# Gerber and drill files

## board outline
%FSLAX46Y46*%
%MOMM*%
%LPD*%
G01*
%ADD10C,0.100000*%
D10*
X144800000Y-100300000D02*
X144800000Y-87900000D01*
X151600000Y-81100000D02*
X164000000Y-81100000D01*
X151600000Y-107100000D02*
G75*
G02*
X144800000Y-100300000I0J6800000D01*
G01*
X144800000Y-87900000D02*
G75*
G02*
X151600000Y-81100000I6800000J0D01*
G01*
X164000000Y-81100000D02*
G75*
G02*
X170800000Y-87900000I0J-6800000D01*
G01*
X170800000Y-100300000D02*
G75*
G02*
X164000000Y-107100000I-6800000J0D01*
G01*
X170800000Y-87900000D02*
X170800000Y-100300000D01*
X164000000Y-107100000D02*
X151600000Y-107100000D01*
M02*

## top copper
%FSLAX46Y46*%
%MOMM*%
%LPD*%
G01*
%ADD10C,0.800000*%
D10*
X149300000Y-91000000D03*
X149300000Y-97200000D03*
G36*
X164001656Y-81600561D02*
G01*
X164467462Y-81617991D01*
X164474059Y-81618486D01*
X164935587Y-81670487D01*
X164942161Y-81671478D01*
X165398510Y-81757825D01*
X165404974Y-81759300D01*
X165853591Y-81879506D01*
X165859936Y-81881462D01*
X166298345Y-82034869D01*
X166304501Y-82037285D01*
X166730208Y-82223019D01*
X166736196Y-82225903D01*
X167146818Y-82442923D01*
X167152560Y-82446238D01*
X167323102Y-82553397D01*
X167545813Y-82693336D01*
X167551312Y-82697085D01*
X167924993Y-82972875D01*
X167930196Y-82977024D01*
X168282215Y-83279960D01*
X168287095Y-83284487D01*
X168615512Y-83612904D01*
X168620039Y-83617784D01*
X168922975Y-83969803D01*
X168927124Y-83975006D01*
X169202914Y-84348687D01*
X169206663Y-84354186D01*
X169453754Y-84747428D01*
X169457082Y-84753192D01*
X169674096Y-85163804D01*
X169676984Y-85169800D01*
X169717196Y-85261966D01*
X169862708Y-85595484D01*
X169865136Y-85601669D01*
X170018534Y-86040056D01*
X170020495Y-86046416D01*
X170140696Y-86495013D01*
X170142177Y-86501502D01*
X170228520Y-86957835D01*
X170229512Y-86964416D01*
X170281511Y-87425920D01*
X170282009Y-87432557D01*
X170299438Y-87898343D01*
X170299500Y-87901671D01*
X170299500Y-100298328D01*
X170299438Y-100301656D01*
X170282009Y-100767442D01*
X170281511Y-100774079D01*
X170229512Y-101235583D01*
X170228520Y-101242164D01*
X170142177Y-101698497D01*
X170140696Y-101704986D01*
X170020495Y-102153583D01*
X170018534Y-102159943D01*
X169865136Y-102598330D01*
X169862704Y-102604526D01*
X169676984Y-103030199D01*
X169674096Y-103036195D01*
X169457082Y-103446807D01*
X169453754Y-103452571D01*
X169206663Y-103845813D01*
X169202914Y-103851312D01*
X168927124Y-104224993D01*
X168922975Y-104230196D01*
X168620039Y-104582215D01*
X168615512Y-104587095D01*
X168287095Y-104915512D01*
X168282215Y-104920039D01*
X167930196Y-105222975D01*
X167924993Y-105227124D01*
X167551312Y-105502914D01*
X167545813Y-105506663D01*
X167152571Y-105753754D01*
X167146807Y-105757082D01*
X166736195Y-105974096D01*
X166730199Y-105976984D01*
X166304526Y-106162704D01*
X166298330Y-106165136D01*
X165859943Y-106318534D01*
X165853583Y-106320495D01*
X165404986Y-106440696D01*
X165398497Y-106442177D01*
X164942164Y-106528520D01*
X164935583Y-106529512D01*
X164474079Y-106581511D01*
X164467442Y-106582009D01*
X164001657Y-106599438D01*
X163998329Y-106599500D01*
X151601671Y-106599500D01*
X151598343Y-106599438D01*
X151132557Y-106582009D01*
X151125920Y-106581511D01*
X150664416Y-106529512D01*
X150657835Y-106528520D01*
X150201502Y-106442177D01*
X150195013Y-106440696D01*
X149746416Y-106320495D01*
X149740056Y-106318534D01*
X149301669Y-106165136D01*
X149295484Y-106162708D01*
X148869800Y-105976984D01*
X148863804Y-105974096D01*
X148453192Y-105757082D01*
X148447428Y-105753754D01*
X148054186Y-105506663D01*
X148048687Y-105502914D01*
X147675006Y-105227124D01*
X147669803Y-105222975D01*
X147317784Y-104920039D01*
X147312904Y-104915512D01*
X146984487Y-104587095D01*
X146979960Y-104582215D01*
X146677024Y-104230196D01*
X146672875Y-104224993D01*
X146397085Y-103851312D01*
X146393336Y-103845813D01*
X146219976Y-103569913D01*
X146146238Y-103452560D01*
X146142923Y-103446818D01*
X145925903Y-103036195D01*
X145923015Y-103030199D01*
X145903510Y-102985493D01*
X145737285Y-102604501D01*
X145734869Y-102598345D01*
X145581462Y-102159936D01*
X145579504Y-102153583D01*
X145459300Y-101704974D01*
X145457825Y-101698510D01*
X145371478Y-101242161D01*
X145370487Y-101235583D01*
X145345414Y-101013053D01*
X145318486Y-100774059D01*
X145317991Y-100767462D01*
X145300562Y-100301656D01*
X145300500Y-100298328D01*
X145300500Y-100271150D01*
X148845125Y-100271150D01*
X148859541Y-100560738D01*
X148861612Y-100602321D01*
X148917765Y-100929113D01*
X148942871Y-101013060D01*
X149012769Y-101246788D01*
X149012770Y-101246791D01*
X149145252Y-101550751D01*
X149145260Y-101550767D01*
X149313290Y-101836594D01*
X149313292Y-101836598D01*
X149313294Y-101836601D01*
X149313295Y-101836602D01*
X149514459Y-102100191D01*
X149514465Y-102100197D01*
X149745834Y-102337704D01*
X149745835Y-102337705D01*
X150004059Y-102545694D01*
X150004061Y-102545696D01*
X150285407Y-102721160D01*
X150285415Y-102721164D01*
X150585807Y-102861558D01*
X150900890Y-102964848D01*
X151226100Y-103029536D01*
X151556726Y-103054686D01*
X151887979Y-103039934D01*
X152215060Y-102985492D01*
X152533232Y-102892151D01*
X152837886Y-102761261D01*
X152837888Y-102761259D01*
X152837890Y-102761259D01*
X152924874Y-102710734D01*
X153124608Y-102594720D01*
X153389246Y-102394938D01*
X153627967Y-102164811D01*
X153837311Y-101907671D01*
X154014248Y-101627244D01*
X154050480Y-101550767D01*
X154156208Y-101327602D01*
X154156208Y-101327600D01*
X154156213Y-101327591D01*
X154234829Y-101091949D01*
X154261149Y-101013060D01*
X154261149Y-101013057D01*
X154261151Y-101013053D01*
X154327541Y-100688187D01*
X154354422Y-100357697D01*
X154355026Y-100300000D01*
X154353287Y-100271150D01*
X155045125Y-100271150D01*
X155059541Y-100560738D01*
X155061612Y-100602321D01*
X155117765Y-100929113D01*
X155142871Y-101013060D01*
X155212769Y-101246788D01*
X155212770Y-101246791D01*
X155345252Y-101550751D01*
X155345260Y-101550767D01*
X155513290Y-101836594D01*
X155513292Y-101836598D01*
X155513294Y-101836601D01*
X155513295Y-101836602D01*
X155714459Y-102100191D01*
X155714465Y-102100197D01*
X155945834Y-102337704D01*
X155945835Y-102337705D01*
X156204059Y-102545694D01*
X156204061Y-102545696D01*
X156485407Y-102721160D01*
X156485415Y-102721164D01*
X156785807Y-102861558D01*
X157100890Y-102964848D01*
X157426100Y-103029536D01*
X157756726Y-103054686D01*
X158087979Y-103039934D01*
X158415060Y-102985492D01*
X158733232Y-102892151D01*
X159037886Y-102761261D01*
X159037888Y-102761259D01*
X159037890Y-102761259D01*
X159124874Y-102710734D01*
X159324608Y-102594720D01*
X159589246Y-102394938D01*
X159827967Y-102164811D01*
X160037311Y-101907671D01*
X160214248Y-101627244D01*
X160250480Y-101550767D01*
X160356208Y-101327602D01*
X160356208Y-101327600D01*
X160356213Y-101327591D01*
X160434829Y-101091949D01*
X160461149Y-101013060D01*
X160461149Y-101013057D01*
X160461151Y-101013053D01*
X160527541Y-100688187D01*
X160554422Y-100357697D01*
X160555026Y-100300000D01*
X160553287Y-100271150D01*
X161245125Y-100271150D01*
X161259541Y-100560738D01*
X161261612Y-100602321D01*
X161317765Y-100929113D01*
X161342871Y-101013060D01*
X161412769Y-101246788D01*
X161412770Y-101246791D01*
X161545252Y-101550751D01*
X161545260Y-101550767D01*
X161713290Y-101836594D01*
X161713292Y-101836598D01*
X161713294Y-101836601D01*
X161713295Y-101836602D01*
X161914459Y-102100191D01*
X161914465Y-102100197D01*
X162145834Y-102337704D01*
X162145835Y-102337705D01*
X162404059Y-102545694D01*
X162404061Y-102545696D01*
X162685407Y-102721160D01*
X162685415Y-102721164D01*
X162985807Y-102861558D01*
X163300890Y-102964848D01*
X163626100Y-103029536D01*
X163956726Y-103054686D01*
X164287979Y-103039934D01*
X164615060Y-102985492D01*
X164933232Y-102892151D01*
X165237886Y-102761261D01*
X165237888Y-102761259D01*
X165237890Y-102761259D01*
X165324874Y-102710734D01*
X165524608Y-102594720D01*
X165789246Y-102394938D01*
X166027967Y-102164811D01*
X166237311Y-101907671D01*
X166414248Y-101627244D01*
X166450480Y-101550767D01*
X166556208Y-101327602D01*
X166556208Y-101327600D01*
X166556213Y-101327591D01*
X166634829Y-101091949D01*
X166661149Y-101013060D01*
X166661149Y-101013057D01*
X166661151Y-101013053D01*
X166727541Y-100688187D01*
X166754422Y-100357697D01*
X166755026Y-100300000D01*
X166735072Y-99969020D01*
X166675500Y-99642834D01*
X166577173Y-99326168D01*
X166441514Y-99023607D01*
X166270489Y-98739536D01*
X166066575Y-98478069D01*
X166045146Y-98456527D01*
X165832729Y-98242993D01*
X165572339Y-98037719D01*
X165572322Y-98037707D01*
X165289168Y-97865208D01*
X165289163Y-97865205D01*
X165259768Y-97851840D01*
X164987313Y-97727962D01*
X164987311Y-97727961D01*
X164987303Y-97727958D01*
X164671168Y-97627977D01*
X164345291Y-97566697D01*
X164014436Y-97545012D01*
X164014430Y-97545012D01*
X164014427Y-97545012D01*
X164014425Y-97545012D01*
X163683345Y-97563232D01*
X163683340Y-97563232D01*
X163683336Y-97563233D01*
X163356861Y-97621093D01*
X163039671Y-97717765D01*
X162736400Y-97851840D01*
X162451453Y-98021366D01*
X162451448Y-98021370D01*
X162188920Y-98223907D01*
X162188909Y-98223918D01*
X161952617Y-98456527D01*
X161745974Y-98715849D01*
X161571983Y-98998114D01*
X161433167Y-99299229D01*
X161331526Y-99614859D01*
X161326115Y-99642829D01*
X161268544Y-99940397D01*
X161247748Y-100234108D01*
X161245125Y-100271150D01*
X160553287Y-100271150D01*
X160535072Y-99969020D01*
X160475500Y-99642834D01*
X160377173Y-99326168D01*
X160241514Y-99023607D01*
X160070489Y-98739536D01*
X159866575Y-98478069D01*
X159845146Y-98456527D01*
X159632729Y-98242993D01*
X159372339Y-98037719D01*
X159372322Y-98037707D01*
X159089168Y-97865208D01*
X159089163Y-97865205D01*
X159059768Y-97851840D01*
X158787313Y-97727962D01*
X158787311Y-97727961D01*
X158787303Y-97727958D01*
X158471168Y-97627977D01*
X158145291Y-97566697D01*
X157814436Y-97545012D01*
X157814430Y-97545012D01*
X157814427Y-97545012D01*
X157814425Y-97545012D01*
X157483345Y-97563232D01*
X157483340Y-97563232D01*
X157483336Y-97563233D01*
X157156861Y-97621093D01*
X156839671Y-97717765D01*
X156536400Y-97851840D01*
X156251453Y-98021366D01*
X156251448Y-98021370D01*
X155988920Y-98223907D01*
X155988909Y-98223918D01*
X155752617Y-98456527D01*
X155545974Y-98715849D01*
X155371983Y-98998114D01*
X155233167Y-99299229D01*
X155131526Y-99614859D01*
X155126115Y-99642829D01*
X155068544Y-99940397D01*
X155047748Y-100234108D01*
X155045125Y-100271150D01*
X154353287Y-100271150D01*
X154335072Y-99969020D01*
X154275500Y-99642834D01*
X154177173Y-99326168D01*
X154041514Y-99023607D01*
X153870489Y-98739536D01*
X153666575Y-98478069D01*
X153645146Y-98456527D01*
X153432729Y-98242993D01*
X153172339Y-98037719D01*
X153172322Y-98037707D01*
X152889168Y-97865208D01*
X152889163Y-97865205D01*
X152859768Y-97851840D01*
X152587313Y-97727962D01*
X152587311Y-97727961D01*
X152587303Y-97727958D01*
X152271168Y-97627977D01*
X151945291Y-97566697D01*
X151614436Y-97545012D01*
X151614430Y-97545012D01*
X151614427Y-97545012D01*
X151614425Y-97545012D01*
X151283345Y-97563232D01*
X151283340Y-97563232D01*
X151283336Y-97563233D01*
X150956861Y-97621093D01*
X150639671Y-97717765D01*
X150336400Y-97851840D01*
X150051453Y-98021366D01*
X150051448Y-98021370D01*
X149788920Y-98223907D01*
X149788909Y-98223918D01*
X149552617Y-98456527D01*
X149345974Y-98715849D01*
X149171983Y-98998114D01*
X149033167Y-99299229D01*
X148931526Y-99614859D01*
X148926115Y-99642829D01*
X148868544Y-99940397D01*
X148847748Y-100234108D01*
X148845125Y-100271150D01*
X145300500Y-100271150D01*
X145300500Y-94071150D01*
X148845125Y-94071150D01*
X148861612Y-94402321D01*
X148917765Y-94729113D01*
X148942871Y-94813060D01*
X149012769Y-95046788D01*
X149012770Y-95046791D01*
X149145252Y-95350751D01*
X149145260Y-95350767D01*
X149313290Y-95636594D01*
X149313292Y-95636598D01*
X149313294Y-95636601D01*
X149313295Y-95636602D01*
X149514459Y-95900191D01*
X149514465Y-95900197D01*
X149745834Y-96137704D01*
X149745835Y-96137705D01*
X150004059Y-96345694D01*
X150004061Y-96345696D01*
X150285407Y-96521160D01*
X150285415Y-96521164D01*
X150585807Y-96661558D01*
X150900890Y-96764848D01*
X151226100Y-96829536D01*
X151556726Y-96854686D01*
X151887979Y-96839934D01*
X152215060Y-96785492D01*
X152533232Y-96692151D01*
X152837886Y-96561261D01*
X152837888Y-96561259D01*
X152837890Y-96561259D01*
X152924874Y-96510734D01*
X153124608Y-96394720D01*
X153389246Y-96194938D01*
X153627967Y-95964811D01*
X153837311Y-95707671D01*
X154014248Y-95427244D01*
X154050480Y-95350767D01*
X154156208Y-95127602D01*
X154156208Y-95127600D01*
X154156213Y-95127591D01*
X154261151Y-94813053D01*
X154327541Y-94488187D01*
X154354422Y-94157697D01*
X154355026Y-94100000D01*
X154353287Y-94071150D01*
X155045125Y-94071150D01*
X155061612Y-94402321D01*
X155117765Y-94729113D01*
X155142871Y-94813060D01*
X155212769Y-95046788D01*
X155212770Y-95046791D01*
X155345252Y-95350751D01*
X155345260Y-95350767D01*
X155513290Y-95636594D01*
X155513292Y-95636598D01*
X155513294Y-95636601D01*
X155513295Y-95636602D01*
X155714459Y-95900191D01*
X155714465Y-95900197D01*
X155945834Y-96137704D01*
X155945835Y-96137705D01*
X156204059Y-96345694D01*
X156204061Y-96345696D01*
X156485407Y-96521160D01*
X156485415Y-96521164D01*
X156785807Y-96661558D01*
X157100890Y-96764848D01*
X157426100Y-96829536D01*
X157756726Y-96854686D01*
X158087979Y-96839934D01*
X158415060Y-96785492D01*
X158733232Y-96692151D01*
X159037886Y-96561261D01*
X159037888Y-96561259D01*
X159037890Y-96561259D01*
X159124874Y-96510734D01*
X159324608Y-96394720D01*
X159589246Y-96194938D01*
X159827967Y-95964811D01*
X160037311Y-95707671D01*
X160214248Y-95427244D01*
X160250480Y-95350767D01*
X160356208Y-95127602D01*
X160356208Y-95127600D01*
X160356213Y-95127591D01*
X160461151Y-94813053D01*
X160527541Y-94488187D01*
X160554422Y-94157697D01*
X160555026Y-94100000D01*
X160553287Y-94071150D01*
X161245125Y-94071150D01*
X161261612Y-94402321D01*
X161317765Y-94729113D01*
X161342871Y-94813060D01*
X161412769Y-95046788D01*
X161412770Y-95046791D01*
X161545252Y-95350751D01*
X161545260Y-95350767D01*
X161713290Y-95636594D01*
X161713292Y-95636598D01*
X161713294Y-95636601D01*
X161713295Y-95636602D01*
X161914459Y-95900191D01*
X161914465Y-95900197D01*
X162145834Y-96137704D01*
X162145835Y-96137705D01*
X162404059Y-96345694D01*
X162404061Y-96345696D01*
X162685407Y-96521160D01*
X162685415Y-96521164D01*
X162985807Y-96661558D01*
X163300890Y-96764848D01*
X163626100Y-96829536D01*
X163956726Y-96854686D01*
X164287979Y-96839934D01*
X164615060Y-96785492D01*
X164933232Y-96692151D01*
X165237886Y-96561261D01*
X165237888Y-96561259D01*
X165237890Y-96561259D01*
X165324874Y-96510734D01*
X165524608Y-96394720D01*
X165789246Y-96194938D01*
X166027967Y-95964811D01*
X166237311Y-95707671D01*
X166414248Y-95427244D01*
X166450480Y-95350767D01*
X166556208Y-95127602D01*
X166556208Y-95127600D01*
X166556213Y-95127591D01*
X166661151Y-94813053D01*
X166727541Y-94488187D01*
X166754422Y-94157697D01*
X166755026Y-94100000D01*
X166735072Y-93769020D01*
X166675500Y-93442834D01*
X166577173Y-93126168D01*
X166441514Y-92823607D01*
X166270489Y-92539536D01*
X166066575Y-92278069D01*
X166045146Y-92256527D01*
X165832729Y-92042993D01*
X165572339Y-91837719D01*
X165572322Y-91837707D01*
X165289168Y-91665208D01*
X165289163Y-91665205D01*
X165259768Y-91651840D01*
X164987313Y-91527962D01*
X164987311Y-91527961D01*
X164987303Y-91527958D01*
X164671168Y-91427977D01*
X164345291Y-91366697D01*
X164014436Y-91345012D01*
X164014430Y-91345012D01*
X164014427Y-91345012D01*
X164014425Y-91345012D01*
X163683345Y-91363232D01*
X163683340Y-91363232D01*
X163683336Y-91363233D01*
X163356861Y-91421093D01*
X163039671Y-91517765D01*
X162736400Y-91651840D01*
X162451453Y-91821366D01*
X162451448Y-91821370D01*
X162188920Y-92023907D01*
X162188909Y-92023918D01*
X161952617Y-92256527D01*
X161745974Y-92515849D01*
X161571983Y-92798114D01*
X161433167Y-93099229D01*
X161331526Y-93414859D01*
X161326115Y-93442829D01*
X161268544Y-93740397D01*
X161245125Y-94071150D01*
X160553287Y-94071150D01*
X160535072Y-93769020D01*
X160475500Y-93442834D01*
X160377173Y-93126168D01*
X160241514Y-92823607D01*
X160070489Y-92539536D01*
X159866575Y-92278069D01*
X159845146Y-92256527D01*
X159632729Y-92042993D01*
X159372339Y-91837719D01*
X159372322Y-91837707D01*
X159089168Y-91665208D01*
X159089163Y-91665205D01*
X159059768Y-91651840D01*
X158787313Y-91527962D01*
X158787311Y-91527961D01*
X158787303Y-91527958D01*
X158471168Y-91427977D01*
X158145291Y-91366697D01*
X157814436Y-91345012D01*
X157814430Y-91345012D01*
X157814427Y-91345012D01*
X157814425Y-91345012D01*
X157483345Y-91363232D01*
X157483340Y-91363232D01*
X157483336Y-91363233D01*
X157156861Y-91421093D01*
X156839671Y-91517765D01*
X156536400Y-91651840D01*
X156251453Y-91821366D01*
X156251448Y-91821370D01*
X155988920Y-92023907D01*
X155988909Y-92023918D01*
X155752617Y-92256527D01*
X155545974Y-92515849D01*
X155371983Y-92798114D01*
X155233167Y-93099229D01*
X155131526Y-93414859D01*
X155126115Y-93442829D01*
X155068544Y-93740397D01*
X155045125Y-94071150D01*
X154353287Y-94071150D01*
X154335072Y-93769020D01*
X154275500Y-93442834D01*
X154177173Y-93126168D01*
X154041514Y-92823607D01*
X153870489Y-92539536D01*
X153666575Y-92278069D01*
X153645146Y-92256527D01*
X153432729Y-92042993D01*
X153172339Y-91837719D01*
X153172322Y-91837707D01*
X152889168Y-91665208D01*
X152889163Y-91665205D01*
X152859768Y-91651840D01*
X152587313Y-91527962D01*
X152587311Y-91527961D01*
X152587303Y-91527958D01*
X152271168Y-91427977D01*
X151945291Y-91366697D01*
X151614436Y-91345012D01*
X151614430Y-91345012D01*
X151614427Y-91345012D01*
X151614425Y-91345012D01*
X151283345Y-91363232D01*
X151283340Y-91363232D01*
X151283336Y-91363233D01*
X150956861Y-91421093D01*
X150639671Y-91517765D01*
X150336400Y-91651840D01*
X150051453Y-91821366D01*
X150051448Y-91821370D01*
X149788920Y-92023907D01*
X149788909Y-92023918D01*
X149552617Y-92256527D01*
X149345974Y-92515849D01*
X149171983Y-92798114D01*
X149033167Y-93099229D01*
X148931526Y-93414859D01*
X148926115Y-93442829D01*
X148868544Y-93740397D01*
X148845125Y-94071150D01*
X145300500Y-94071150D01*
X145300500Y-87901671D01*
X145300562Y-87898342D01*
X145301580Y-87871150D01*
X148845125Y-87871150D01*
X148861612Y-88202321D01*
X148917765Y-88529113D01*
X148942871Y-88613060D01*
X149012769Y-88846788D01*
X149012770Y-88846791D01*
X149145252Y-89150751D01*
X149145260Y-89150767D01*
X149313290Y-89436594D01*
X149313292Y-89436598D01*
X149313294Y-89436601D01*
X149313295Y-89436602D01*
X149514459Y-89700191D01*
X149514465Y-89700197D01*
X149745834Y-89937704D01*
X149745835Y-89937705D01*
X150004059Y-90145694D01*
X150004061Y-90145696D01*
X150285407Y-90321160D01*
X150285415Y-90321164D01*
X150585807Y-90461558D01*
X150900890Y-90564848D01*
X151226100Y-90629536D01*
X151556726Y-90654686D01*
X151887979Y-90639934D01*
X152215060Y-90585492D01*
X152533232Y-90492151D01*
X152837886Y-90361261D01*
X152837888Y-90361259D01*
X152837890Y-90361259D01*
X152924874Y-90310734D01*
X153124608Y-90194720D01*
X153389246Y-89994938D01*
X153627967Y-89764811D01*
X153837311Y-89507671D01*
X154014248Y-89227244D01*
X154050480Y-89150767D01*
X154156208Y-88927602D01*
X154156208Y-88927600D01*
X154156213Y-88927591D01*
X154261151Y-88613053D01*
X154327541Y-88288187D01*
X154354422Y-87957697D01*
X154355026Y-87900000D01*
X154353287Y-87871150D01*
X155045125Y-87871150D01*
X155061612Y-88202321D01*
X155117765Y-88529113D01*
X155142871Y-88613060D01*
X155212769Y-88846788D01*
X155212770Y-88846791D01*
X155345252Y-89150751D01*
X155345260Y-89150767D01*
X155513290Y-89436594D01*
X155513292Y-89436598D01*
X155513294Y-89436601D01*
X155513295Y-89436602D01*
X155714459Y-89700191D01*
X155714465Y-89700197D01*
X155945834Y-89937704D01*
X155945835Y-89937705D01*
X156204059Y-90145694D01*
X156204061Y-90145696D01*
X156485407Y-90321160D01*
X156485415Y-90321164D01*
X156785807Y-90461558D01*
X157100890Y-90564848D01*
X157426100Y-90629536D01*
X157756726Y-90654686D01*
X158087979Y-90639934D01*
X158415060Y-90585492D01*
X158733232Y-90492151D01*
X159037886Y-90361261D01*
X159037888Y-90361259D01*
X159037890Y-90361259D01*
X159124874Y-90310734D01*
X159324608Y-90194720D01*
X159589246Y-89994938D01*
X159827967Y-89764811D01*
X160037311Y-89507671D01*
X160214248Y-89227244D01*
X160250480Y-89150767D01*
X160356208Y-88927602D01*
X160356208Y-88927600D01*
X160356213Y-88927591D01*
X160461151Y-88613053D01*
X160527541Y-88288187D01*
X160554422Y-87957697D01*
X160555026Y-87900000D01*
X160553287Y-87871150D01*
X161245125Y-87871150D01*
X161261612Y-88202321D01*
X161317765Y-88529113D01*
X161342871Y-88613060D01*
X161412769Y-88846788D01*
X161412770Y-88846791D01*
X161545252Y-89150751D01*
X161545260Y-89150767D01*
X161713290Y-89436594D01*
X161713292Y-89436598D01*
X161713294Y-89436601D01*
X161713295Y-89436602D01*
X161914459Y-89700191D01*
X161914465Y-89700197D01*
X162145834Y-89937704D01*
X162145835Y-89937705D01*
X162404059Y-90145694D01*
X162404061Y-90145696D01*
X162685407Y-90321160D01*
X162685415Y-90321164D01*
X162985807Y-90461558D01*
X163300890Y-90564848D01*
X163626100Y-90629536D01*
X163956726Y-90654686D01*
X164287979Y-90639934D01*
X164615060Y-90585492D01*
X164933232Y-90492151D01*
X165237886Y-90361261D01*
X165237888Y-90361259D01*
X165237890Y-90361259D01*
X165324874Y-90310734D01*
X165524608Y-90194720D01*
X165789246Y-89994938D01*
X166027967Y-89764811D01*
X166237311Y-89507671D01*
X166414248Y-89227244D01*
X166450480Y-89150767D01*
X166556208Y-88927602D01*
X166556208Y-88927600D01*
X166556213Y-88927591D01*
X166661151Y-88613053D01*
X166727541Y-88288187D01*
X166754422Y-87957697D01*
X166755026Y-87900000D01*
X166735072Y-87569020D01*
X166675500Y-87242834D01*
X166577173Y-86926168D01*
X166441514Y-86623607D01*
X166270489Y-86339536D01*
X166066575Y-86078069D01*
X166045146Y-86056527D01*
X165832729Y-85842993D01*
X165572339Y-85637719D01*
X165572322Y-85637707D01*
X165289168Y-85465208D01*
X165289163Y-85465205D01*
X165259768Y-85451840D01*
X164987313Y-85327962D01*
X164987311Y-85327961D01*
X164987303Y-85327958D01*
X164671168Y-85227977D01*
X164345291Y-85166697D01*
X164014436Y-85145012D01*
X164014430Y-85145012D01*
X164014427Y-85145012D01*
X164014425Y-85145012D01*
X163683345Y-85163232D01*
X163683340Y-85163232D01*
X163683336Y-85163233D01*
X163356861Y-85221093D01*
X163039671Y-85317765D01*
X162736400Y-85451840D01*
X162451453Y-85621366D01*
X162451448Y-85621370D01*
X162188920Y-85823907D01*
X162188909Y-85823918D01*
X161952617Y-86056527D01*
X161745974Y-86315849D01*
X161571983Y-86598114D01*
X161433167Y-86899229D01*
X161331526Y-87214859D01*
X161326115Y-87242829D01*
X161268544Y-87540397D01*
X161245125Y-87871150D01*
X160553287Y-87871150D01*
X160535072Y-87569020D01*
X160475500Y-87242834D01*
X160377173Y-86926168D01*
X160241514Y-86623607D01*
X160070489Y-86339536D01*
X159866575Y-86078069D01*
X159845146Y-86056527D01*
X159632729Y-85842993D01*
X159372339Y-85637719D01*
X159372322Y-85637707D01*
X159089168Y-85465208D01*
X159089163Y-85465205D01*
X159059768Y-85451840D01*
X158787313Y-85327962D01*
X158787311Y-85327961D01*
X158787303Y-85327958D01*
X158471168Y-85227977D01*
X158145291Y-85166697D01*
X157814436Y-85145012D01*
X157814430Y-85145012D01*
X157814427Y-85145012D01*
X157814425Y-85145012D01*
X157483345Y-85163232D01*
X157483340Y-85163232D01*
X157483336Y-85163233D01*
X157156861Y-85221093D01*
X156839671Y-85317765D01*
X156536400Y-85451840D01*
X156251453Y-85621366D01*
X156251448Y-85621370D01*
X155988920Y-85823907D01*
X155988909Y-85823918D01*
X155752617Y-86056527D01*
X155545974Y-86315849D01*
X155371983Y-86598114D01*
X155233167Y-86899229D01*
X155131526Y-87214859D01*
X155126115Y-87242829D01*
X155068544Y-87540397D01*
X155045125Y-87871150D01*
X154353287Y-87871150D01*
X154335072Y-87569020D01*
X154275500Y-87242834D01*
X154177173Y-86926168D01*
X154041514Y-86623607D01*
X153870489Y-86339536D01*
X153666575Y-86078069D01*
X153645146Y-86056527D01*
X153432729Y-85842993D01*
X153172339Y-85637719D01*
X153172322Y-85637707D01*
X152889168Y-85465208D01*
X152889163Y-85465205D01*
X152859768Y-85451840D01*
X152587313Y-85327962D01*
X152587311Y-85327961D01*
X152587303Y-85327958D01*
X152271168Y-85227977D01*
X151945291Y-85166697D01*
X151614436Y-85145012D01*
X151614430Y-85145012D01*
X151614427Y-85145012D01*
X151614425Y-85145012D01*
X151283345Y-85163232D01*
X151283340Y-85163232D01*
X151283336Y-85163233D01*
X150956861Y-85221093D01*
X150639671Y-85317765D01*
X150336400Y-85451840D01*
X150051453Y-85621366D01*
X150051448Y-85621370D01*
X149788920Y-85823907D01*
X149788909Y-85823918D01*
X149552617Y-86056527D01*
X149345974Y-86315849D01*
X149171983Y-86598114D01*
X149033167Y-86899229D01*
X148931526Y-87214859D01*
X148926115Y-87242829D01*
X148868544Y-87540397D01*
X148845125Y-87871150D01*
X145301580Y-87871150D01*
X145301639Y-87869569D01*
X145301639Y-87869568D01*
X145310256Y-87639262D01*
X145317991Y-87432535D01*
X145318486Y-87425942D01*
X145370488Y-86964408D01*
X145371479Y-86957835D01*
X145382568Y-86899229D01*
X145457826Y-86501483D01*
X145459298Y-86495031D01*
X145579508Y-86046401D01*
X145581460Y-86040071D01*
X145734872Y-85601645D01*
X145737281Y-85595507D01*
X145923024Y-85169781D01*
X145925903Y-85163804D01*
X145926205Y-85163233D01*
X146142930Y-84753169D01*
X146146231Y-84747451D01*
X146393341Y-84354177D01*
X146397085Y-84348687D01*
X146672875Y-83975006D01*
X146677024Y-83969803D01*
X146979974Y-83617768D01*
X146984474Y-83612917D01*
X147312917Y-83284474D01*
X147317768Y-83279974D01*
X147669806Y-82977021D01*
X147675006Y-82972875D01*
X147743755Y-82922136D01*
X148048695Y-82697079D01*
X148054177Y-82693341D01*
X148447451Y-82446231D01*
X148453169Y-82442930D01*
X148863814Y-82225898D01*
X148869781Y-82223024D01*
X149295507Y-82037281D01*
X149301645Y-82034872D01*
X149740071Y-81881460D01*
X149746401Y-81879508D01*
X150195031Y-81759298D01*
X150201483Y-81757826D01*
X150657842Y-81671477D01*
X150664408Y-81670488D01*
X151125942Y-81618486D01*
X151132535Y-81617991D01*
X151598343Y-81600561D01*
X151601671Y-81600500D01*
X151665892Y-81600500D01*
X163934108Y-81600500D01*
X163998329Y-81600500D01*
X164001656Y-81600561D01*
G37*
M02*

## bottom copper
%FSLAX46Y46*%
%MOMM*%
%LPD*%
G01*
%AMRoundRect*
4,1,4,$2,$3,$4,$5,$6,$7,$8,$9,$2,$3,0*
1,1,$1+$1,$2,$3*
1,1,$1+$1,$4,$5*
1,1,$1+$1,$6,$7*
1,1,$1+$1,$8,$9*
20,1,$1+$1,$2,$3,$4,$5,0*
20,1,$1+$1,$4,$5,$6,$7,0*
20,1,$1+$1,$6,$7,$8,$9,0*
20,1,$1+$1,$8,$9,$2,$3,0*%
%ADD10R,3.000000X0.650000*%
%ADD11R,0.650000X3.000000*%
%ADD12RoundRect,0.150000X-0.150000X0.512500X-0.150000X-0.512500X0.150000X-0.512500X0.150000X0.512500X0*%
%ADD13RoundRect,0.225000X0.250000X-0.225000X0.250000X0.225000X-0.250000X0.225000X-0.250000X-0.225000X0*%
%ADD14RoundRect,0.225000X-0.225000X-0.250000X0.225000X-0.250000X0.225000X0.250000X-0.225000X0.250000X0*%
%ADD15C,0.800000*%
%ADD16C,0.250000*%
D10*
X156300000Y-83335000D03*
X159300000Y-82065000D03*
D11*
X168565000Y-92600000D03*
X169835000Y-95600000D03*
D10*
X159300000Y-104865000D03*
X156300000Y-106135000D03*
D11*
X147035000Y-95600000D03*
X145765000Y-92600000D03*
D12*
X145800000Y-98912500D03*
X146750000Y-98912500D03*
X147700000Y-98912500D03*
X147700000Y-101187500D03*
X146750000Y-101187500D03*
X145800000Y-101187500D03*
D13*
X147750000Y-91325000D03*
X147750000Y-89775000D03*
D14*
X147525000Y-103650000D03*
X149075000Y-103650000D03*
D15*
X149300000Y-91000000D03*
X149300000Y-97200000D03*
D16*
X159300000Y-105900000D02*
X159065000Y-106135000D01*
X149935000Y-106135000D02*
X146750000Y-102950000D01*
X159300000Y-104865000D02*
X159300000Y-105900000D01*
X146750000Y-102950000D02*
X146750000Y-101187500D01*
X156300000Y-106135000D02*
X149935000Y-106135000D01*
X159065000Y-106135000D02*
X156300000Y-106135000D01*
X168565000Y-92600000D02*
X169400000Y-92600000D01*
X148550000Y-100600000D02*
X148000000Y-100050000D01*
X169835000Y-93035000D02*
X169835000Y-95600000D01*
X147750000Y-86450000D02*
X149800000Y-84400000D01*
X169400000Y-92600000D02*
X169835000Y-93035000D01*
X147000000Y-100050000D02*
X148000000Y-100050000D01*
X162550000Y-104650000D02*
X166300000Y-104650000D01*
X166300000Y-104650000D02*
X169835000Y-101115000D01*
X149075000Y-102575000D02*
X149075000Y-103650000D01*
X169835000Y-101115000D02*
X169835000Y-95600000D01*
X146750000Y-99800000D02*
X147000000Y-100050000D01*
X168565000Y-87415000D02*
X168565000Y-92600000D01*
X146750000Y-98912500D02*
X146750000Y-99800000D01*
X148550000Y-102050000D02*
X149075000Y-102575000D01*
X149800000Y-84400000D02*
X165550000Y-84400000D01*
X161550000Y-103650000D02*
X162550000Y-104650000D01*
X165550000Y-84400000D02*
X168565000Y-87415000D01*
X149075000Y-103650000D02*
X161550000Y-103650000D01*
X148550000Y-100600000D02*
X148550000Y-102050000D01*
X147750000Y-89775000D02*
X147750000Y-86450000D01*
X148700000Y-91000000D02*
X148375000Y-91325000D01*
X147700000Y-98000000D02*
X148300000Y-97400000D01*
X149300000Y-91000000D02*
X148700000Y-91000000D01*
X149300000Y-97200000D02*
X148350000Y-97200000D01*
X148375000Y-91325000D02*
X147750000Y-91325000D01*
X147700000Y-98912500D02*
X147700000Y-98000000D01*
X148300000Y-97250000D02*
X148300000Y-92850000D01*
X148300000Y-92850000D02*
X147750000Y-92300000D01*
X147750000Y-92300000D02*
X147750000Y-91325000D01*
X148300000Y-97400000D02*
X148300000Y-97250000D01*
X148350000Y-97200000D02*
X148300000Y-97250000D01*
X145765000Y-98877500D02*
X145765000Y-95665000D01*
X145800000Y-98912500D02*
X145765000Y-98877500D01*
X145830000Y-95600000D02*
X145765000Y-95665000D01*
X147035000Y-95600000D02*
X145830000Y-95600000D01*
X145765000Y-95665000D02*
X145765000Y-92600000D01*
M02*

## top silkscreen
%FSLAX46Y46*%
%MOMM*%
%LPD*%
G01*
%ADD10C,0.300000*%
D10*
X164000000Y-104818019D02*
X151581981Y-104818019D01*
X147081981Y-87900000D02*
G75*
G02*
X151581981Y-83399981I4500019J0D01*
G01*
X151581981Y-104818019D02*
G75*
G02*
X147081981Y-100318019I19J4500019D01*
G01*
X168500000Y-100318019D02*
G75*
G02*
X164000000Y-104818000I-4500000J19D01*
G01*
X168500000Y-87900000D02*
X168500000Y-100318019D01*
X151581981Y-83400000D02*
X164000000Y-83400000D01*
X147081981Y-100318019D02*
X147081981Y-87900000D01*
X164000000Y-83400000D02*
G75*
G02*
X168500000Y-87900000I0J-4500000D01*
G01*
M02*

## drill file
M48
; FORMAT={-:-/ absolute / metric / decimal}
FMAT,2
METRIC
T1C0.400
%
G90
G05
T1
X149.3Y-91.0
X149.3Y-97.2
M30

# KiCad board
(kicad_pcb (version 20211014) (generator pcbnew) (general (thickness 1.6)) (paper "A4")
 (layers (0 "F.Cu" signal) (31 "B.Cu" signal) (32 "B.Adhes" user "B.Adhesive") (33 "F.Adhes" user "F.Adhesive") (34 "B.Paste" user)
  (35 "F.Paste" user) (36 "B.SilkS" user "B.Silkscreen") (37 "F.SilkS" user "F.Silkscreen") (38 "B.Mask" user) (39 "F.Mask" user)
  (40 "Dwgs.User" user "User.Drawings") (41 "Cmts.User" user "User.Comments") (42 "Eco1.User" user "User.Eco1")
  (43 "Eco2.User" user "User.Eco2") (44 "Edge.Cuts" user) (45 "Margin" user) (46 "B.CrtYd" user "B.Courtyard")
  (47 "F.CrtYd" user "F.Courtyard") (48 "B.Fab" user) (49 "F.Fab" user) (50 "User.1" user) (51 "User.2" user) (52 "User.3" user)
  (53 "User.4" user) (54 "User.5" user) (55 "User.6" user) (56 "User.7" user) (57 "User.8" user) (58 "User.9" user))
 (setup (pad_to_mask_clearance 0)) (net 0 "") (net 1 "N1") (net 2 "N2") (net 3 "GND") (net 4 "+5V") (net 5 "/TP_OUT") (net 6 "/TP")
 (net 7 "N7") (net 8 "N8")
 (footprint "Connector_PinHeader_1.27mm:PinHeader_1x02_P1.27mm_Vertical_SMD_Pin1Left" (layer "B.Cu") (at 157.8 82.7)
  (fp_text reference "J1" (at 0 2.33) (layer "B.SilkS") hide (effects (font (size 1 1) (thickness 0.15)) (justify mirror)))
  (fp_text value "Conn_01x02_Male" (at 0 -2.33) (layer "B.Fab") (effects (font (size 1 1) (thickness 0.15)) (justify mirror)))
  (pad "1" smd rect (at -1.5 0.635) (size 3 0.65) (layers "B.Cu" "B.Paste" "B.Mask") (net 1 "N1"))
  (pad "2" smd rect (at 1.5 -0.635) (size 3 0.65) (layers "B.Cu" "B.Paste" "B.Mask") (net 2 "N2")))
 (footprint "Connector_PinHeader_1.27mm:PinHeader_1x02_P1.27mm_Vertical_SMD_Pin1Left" (layer "B.Cu") (at 169.2 94.1 -90)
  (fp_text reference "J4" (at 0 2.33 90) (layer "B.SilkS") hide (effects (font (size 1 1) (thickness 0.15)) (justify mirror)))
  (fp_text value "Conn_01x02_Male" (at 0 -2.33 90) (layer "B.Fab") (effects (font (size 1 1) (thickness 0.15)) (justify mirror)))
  (pad "1" smd rect (at -1.5 0.635 270) (size 3 0.65) (layers "B.Cu" "B.Paste" "B.Mask") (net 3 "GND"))
  (pad "2" smd rect (at 1.5 -0.635 270) (size 3 0.65) (layers "B.Cu" "B.Paste" "B.Mask") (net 3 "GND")))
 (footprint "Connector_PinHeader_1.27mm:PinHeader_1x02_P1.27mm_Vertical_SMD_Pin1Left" (layer "B.Cu") (at 157.8 105.5 180)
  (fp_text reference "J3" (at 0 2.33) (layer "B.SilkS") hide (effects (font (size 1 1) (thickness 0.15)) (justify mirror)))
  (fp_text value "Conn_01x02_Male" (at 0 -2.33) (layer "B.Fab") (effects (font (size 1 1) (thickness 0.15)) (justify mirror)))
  (pad "1" smd rect (at -1.5 0.635 180) (size 3 0.65) (layers "B.Cu" "B.Paste" "B.Mask") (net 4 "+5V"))
  (pad "2" smd rect (at 1.5 -0.635 180) (size 3 0.65) (layers "B.Cu" "B.Paste" "B.Mask") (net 4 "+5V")))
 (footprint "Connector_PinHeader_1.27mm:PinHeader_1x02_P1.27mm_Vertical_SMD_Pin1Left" (layer "B.Cu") (at 146.4 94.1 90)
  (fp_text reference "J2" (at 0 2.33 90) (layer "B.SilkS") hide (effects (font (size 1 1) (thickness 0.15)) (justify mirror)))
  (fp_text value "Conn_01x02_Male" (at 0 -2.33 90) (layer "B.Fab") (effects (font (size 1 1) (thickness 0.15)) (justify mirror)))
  (pad "1" smd rect (at -1.5 0.635 90) (size 3 0.65) (layers "B.Cu" "B.Paste" "B.Mask") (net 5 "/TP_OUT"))
  (pad "2" smd rect (at 1.5 -0.635 90) (size 3 0.65) (layers "B.Cu" "B.Paste" "B.Mask") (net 5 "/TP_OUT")))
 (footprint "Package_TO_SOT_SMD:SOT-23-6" (layer "B.Cu") (at 146.75 100.05 -90)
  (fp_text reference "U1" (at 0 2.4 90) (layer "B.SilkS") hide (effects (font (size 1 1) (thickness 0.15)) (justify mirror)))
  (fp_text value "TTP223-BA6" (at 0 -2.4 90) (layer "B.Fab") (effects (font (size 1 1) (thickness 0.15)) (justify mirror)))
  (pad "1" smd roundrect (at -1.1375 0.95 270) (size 1.325 0.6) (layers "B.Cu" "B.Paste" "B.Mask") (roundrect_rratio 0.25) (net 5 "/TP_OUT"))
  (pad "2" smd roundrect (at -1.1375 0 270) (size 1.325 0.6) (layers "B.Cu" "B.Paste" "B.Mask") (roundrect_rratio 0.25) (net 3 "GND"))
  (pad "3" smd roundrect (at -1.1375 -0.95 270) (size 1.325 0.6) (layers "B.Cu" "B.Paste" "B.Mask") (roundrect_rratio 0.25) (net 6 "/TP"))
  (pad "4" smd roundrect (at 1.1375 -0.95 270) (size 1.325 0.6) (layers "B.Cu" "B.Paste" "B.Mask") (roundrect_rratio 0.25) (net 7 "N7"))
  (pad "5" smd roundrect (at 1.1375 0 270) (size 1.325 0.6) (layers "B.Cu" "B.Paste" "B.Mask") (roundrect_rratio 0.25) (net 4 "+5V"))
  (pad "6" smd roundrect (at 1.1375 0.95 270) (size 1.325 0.6) (layers "B.Cu" "B.Paste" "B.Mask") (roundrect_rratio 0.25) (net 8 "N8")))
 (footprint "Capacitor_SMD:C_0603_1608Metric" (layer "B.Cu") (at 147.75 90.55 90)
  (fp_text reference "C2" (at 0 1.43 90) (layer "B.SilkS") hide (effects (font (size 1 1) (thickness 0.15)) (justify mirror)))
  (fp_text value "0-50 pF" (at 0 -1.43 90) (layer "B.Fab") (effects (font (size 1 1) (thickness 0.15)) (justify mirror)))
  (pad "1" smd roundrect (at -0.775 0 90) (size 0.9 0.95) (layers "B.Cu" "B.Paste" "B.Mask") (roundrect_rratio 0.25) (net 6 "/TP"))
  (pad "2" smd roundrect (at 0.775 0 90) (size 0.9 0.95) (layers "B.Cu" "B.Paste" "B.Mask") (roundrect_rratio 0.25) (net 3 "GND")))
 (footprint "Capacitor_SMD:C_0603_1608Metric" (layer "B.Cu") (at 148.3 103.65)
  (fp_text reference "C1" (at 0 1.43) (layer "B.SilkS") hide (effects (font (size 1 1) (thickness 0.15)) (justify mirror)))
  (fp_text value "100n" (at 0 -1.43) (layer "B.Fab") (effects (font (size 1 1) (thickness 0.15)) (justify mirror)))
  (pad "1" smd roundrect (at -0.775 0) (size 0.9 0.95) (layers "B.Cu" "B.Paste" "B.Mask") (roundrect_rratio 0.25) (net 4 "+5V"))
  (pad "2" smd roundrect (at 0.775 0) (size 0.9 0.95) (layers "B.Cu" "B.Paste" "B.Mask") (roundrect_rratio 0.25) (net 3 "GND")))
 (gr_line (start 164 104.818019) (end 151.581981 104.818019) (layer "F.SilkS") (width 0.3))
 (gr_arc (start 147.081981 87.9) (mid 148.399999 84.718013) (end 151.581981 83.4) (layer "F.SilkS") (width 0.3))
 (gr_arc (start 151.581981 104.818019) (mid 148.400006 103.499994) (end 147.081981 100.318019) (layer "F.SilkS") (width 0.3))
 (gr_arc (start 168.5 100.318019) (mid 167.181981 103.5) (end 164 104.818019) (layer "F.SilkS") (width 0.3))
 (gr_line (start 168.5 87.9) (end 168.5 100.318019) (layer "F.SilkS") (width 0.3))
 (gr_line (start 151.581981 83.4) (end 164 83.4) (layer "F.SilkS") (width 0.3))
 (gr_line (start 147.081981 100.318019) (end 147.081981 87.9) (layer "F.SilkS") (width 0.3))
 (gr_arc (start 164 83.4) (mid 167.181981 84.718019) (end 168.5 87.9) (layer "F.SilkS") (width 0.3))
 (gr_line (start 144.8 100.3) (end 144.8 87.9) (layer "Edge.Cuts") (width 0.1))
 (gr_line (start 151.6 81.1) (end 164 81.1) (layer "Edge.Cuts") (width 0.1))
 (gr_arc (start 151.6 107.1) (mid 146.791674 105.108326) (end 144.8 100.3) (layer "Edge.Cuts") (width 0.1))
 (gr_arc (start 144.8 87.9) (mid 146.791674 83.091674) (end 151.6 81.1) (layer "Edge.Cuts") (width 0.1))
 (gr_arc (start 164 81.1) (mid 168.808326 83.091674) (end 170.8 87.9) (layer "Edge.Cuts") (width 0.1))
 (gr_arc (start 170.8 100.3) (mid 168.808326 105.108326) (end 164 107.1) (layer "Edge.Cuts") (width 0.1))
 (gr_line (start 170.8 87.9) (end 170.8 100.3) (layer "Edge.Cuts") (width 0.1))
 (gr_line (start 164 107.1) (end 151.6 107.1) (layer "Edge.Cuts") (width 0.1))
 (segment (start 159.3 105.9) (end 159.065 106.135) (width 0.25) (layer "B.Cu") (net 4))
 (segment (start 149.935 106.135) (end 146.75 102.95) (width 0.25) (layer "B.Cu") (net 4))
 (segment (start 159.3 104.865) (end 159.3 105.9) (width 0.25) (layer "B.Cu") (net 4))
 (segment (start 146.75 102.95) (end 146.75 101.1875) (width 0.25) (layer "B.Cu") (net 4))
 (segment (start 156.3 106.135) (end 149.935 106.135) (width 0.25) (layer "B.Cu") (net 4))
 (segment (start 159.065 106.135) (end 156.3 106.135) (width 0.25) (layer "B.Cu") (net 4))
 (segment (start 168.565 92.6) (end 169.4 92.6) (width 0.25) (layer "B.Cu") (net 3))
 (segment (start 148.55 100.6) (end 148 100.05) (width 0.25) (layer "B.Cu") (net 3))
 (segment (start 169.835 93.035) (end 169.835 95.6) (width 0.25) (layer "B.Cu") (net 3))
 (segment (start 147.75 86.45) (end 149.8 84.4) (width 0.25) (layer "B.Cu") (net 3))
 (segment (start 169.4 92.6) (end 169.835 93.035) (width 0.25) (layer "B.Cu") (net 3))
 (segment (start 147 100.05) (end 148 100.05) (width 0.25) (layer "B.Cu") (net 3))
 (segment (start 162.55 104.65) (end 166.3 104.65) (width 0.25) (layer "B.Cu") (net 3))
 (segment (start 166.3 104.65) (end 169.835 101.115) (width 0.25) (layer "B.Cu") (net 3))
 (segment (start 149.075 102.575) (end 149.075 103.65) (width 0.25) (layer "B.Cu") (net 3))
 (segment (start 169.835 101.115) (end 169.835 95.6) (width 0.25) (layer "B.Cu") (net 3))
 (segment (start 146.75 99.8) (end 147 100.05) (width 0.25) (layer "B.Cu") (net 3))
 (segment (start 168.565 87.415) (end 168.565 92.6) (width 0.25) (layer "B.Cu") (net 3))
 (segment (start 146.75 98.9125) (end 146.75 99.8) (width 0.25) (layer "B.Cu") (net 3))
 (segment (start 148.55 102.05) (end 149.075 102.575) (width 0.25) (layer "B.Cu") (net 3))
 (segment (start 149.8 84.4) (end 165.55 84.4) (width 0.25) (layer "B.Cu") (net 3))
 (segment (start 161.55 103.65) (end 162.55 104.65) (width 0.25) (layer "B.Cu") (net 3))
 (segment (start 165.55 84.4) (end 168.565 87.415) (width 0.25) (layer "B.Cu") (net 3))
 (segment (start 149.075 103.65) (end 161.55 103.65) (width 0.25) (layer "B.Cu") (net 3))
 (segment (start 148.55 100.6) (end 148.55 102.05) (width 0.25) (layer "B.Cu") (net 3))
 (segment (start 147.75 89.775) (end 147.75 86.45) (width 0.25) (layer "B.Cu") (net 3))
 (via (at 149.3 91) (size 0.8) (drill 0.4) (layers "F.Cu" "B.Cu") (free) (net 6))
 (via (at 149.3 97.2) (size 0.8) (drill 0.4) (layers "F.Cu" "B.Cu") (free) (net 6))
 (segment (start 148.7 91) (end 148.375 91.325) (width 0.25) (layer "B.Cu") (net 6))
 (segment (start 147.7 98) (end 148.3 97.4) (width 0.25) (layer "B.Cu") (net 6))
 (segment (start 149.3 91) (end 148.7 91) (width 0.25) (layer "B.Cu") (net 6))
 (segment (start 149.3 97.2) (end 148.35 97.2) (width 0.25) (layer "B.Cu") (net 6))
 (segment (start 148.375 91.325) (end 147.75 91.325) (width 0.25) (layer "B.Cu") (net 6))
 (segment (start 147.7 98.9125) (end 147.7 98) (width 0.25) (layer "B.Cu") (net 6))
 (segment (start 148.3 97.25) (end 148.3 92.85) (width 0.25) (layer "B.Cu") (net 6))
 (segment (start 148.3 92.85) (end 147.75 92.3) (width 0.25) (layer "B.Cu") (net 6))
 (segment (start 147.75 92.3) (end 147.75 91.325) (width 0.25) (layer "B.Cu") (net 6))
 (segment (start 148.3 97.4) (end 148.3 97.25) (width 0.25) (layer "B.Cu") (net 6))
 (segment (start 148.35 97.2) (end 148.3 97.25) (width 0.25) (layer "B.Cu") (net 6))
 (segment (start 145.765 98.8775) (end 145.765 95.665) (width 0.25) (layer "B.Cu") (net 5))
 (segment (start 145.8 98.9125) (end 145.765 98.8775) (width 0.25) (layer "B.Cu") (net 5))
 (segment (start 145.83 95.6) (end 145.765 95.665) (width 0.25) (layer "B.Cu") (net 5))
 (segment (start 147.035 95.6) (end 145.83 95.6) (width 0.25) (layer "B.Cu") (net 5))
 (segment (start 145.765 95.665) (end 145.765 92.6) (width 0.25) (layer "B.Cu") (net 5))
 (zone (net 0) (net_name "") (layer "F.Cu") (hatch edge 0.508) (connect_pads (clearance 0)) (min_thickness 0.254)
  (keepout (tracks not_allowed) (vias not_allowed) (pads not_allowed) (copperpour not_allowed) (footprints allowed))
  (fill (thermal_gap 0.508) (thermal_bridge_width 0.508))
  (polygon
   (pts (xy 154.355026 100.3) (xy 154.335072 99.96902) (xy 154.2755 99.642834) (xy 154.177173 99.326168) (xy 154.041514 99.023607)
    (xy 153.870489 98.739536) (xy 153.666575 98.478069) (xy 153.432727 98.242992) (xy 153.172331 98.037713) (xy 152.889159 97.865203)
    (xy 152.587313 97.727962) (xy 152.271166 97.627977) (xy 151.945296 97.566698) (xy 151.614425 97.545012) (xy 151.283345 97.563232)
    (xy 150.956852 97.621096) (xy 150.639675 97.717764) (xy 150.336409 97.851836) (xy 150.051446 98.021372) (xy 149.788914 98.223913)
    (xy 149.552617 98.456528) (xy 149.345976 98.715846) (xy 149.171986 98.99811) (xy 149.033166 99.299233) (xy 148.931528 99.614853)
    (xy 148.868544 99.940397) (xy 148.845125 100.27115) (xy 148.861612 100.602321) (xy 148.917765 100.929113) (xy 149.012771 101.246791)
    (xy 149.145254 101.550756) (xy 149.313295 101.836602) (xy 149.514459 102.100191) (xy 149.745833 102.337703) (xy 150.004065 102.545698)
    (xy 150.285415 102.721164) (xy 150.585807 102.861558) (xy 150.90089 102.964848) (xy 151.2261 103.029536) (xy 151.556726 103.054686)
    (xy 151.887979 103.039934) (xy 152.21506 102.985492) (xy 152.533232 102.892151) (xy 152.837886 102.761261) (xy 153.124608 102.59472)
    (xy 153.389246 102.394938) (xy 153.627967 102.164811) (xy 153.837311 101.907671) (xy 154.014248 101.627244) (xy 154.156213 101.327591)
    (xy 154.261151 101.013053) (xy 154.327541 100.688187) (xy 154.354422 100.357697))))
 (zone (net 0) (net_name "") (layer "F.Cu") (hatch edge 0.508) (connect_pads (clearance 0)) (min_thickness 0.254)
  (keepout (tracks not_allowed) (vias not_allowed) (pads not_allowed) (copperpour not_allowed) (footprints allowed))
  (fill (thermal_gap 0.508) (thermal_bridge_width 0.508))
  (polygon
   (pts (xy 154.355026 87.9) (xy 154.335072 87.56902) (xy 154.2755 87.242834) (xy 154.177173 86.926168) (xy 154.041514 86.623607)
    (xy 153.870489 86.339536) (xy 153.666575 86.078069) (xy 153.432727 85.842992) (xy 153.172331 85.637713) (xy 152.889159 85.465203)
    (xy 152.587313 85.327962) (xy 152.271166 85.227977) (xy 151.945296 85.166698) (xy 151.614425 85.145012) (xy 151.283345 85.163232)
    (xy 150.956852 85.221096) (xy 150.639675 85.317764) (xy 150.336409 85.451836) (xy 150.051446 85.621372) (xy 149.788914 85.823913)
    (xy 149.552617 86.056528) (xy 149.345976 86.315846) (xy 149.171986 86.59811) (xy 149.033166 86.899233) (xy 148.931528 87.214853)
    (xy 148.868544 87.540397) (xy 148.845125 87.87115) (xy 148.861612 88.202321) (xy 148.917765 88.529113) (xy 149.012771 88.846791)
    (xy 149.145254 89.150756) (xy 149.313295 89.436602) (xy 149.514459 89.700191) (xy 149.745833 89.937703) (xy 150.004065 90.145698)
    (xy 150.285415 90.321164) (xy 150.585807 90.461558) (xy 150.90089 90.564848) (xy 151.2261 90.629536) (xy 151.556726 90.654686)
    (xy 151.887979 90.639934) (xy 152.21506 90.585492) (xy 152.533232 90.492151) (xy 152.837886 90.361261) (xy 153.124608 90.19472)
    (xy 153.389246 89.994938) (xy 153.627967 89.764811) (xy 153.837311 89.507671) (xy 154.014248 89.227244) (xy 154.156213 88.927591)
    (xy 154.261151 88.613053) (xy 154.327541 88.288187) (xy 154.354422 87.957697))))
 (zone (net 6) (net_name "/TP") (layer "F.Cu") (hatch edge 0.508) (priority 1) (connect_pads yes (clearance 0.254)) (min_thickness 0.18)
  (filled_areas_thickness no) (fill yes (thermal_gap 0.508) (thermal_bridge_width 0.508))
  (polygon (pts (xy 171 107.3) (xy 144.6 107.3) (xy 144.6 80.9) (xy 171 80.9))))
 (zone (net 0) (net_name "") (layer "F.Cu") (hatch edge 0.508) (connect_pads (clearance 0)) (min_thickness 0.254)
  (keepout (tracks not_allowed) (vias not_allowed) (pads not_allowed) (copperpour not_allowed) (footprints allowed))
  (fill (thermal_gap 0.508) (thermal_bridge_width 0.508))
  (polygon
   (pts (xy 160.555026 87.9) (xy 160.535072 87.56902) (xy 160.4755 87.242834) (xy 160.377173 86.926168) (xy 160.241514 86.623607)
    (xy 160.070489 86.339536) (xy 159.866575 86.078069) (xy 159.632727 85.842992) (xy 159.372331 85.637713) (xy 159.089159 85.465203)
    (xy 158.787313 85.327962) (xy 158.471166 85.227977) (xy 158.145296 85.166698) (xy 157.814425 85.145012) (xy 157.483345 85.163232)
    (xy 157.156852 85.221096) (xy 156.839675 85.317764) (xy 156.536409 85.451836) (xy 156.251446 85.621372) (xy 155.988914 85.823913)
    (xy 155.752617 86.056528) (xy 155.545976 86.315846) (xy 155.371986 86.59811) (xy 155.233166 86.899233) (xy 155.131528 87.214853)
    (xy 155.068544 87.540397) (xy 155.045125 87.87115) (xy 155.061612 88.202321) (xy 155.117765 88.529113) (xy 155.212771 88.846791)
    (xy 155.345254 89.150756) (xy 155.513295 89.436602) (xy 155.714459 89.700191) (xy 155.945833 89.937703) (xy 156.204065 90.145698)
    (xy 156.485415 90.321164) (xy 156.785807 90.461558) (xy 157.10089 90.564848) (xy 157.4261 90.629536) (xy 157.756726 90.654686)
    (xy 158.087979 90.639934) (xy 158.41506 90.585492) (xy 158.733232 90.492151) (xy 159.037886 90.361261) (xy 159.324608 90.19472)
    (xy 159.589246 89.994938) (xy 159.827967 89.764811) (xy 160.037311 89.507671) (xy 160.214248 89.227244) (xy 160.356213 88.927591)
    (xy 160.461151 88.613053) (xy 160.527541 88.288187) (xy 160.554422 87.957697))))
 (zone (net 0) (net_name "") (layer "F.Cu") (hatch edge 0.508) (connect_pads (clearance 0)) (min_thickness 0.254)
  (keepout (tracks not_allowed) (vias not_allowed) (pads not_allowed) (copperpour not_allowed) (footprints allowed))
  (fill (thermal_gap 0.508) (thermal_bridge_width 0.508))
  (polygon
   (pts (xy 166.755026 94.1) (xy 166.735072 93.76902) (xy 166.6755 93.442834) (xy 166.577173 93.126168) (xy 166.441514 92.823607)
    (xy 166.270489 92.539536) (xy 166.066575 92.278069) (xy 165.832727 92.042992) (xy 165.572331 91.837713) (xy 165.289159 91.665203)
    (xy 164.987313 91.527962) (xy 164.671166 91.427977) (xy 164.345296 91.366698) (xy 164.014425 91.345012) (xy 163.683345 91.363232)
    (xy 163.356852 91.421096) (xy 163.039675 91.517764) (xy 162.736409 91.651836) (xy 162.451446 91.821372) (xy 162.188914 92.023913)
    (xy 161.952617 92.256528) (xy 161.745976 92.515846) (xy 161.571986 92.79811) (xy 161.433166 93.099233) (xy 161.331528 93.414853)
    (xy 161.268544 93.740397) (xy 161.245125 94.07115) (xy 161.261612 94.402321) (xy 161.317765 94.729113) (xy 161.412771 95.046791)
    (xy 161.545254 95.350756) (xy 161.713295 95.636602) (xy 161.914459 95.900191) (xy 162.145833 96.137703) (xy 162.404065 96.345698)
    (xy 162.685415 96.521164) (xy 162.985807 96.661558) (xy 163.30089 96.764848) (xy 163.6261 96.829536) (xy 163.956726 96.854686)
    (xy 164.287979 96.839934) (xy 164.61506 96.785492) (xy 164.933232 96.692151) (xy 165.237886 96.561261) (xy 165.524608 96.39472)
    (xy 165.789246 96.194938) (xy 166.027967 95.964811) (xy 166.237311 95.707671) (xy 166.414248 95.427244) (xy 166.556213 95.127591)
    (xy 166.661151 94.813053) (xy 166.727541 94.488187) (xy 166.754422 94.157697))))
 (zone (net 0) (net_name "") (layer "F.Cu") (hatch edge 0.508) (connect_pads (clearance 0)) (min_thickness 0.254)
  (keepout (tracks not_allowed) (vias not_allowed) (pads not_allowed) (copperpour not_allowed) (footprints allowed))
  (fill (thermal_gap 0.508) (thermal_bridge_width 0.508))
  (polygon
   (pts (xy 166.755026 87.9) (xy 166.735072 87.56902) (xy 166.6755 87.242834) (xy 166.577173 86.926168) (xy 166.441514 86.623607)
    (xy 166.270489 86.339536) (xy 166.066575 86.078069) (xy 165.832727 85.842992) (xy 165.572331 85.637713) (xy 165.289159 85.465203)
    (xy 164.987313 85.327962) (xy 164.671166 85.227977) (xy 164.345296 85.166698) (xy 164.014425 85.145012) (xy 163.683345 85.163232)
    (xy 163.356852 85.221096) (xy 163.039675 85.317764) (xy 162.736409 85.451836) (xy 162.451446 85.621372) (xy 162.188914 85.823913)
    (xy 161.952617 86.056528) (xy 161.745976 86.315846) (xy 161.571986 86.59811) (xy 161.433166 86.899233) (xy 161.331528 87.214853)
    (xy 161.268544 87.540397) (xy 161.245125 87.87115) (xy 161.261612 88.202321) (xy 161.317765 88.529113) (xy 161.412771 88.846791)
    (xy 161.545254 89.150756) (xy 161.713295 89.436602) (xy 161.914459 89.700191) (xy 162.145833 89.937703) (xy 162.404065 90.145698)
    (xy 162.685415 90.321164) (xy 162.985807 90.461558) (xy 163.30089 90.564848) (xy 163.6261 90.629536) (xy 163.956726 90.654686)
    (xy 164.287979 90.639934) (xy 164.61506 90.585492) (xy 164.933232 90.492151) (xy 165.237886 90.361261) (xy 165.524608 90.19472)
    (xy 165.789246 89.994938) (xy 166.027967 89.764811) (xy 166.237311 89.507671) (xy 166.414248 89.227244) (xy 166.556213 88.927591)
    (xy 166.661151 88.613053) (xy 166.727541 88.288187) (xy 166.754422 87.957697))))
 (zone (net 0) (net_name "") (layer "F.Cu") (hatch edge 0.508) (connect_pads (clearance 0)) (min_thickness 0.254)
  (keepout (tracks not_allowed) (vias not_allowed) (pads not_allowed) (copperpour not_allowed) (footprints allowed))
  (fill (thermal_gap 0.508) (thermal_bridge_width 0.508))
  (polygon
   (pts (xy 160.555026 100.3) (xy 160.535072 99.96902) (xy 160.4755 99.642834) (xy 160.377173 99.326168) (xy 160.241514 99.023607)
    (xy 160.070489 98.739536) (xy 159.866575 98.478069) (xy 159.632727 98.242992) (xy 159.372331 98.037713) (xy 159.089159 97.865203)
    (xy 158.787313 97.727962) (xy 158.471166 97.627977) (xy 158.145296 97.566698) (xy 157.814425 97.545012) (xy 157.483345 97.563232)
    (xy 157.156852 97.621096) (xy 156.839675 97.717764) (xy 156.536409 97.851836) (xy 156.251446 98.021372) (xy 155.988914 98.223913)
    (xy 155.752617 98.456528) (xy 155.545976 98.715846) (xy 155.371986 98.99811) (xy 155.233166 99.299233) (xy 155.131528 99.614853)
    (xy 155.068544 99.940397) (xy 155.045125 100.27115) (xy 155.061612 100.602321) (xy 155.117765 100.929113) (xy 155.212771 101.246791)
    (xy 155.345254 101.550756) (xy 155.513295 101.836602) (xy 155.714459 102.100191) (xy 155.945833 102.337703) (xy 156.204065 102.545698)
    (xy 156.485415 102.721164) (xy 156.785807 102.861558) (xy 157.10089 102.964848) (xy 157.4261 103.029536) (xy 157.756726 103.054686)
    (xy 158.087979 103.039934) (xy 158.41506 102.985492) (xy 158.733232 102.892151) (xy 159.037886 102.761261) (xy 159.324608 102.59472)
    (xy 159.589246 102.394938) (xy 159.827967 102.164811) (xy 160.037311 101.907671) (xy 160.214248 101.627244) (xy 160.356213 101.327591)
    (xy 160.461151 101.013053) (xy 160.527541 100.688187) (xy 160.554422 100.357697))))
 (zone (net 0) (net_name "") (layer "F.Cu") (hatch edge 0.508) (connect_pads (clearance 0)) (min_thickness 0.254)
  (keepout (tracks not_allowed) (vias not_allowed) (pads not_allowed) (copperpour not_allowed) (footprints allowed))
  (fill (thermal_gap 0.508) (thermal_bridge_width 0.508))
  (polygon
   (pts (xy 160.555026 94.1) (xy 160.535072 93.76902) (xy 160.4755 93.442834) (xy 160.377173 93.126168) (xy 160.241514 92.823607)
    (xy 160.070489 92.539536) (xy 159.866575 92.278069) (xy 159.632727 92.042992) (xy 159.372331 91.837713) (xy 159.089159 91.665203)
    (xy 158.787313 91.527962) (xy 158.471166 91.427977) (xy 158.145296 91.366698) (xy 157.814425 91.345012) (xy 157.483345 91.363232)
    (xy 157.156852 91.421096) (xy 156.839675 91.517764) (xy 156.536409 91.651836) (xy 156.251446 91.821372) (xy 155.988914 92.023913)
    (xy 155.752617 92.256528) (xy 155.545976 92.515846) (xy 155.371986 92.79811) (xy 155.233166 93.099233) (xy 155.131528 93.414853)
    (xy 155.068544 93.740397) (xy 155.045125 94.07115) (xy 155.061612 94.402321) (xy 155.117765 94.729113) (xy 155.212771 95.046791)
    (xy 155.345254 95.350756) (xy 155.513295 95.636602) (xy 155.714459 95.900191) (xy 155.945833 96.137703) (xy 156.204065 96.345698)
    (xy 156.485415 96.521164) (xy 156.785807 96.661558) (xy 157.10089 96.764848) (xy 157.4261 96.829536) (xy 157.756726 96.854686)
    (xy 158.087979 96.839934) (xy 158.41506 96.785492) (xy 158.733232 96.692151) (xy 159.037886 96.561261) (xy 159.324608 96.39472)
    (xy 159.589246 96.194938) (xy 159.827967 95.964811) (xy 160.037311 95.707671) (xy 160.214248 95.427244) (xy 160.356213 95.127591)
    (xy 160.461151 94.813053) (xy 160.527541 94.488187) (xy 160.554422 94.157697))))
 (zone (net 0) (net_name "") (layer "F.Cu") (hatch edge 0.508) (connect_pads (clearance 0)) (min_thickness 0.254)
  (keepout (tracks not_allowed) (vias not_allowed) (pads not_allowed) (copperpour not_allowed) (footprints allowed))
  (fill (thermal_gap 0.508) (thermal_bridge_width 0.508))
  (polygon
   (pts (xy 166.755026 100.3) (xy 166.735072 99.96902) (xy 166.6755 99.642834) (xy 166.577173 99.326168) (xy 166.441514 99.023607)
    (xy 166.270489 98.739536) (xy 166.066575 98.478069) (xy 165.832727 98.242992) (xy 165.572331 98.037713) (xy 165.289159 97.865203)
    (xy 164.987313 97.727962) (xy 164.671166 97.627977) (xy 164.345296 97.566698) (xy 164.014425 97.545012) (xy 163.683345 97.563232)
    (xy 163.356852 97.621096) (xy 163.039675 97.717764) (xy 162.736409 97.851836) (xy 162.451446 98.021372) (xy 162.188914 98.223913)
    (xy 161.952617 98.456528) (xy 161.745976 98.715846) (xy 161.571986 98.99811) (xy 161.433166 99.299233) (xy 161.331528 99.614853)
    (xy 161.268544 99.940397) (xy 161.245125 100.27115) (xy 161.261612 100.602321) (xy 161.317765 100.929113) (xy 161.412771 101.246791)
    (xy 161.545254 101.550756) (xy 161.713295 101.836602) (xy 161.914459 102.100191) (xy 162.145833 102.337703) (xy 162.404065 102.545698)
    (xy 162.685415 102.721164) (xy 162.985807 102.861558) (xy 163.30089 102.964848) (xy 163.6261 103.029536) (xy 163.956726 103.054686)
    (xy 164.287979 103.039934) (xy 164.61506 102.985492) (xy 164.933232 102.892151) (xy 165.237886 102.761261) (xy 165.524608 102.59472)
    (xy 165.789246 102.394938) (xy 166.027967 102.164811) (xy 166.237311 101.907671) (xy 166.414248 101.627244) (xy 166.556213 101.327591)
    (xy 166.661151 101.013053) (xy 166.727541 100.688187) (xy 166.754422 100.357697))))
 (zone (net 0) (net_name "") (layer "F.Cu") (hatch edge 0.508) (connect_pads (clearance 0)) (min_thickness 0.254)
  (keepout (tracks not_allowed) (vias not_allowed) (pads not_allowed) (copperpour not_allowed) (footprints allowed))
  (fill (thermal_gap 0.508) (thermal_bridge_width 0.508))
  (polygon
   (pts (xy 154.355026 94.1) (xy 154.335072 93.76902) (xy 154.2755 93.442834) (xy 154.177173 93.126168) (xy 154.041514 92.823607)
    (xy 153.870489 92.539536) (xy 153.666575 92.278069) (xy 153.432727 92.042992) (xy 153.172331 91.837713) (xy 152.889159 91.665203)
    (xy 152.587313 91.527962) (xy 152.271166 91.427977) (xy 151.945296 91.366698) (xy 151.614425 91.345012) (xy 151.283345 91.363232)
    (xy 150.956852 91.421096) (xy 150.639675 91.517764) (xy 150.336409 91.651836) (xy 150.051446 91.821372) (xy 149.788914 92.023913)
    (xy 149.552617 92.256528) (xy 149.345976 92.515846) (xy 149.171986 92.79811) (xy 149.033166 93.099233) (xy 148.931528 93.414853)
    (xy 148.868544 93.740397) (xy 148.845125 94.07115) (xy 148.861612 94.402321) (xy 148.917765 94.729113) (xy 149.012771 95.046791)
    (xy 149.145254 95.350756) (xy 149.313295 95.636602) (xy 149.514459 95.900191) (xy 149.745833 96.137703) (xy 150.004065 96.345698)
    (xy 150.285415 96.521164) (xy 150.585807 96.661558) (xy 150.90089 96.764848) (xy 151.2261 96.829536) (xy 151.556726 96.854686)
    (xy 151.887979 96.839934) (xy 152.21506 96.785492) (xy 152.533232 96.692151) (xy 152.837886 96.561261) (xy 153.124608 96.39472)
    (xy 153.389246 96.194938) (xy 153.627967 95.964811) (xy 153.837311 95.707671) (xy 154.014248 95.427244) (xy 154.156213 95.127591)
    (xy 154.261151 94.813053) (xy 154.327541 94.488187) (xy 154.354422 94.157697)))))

